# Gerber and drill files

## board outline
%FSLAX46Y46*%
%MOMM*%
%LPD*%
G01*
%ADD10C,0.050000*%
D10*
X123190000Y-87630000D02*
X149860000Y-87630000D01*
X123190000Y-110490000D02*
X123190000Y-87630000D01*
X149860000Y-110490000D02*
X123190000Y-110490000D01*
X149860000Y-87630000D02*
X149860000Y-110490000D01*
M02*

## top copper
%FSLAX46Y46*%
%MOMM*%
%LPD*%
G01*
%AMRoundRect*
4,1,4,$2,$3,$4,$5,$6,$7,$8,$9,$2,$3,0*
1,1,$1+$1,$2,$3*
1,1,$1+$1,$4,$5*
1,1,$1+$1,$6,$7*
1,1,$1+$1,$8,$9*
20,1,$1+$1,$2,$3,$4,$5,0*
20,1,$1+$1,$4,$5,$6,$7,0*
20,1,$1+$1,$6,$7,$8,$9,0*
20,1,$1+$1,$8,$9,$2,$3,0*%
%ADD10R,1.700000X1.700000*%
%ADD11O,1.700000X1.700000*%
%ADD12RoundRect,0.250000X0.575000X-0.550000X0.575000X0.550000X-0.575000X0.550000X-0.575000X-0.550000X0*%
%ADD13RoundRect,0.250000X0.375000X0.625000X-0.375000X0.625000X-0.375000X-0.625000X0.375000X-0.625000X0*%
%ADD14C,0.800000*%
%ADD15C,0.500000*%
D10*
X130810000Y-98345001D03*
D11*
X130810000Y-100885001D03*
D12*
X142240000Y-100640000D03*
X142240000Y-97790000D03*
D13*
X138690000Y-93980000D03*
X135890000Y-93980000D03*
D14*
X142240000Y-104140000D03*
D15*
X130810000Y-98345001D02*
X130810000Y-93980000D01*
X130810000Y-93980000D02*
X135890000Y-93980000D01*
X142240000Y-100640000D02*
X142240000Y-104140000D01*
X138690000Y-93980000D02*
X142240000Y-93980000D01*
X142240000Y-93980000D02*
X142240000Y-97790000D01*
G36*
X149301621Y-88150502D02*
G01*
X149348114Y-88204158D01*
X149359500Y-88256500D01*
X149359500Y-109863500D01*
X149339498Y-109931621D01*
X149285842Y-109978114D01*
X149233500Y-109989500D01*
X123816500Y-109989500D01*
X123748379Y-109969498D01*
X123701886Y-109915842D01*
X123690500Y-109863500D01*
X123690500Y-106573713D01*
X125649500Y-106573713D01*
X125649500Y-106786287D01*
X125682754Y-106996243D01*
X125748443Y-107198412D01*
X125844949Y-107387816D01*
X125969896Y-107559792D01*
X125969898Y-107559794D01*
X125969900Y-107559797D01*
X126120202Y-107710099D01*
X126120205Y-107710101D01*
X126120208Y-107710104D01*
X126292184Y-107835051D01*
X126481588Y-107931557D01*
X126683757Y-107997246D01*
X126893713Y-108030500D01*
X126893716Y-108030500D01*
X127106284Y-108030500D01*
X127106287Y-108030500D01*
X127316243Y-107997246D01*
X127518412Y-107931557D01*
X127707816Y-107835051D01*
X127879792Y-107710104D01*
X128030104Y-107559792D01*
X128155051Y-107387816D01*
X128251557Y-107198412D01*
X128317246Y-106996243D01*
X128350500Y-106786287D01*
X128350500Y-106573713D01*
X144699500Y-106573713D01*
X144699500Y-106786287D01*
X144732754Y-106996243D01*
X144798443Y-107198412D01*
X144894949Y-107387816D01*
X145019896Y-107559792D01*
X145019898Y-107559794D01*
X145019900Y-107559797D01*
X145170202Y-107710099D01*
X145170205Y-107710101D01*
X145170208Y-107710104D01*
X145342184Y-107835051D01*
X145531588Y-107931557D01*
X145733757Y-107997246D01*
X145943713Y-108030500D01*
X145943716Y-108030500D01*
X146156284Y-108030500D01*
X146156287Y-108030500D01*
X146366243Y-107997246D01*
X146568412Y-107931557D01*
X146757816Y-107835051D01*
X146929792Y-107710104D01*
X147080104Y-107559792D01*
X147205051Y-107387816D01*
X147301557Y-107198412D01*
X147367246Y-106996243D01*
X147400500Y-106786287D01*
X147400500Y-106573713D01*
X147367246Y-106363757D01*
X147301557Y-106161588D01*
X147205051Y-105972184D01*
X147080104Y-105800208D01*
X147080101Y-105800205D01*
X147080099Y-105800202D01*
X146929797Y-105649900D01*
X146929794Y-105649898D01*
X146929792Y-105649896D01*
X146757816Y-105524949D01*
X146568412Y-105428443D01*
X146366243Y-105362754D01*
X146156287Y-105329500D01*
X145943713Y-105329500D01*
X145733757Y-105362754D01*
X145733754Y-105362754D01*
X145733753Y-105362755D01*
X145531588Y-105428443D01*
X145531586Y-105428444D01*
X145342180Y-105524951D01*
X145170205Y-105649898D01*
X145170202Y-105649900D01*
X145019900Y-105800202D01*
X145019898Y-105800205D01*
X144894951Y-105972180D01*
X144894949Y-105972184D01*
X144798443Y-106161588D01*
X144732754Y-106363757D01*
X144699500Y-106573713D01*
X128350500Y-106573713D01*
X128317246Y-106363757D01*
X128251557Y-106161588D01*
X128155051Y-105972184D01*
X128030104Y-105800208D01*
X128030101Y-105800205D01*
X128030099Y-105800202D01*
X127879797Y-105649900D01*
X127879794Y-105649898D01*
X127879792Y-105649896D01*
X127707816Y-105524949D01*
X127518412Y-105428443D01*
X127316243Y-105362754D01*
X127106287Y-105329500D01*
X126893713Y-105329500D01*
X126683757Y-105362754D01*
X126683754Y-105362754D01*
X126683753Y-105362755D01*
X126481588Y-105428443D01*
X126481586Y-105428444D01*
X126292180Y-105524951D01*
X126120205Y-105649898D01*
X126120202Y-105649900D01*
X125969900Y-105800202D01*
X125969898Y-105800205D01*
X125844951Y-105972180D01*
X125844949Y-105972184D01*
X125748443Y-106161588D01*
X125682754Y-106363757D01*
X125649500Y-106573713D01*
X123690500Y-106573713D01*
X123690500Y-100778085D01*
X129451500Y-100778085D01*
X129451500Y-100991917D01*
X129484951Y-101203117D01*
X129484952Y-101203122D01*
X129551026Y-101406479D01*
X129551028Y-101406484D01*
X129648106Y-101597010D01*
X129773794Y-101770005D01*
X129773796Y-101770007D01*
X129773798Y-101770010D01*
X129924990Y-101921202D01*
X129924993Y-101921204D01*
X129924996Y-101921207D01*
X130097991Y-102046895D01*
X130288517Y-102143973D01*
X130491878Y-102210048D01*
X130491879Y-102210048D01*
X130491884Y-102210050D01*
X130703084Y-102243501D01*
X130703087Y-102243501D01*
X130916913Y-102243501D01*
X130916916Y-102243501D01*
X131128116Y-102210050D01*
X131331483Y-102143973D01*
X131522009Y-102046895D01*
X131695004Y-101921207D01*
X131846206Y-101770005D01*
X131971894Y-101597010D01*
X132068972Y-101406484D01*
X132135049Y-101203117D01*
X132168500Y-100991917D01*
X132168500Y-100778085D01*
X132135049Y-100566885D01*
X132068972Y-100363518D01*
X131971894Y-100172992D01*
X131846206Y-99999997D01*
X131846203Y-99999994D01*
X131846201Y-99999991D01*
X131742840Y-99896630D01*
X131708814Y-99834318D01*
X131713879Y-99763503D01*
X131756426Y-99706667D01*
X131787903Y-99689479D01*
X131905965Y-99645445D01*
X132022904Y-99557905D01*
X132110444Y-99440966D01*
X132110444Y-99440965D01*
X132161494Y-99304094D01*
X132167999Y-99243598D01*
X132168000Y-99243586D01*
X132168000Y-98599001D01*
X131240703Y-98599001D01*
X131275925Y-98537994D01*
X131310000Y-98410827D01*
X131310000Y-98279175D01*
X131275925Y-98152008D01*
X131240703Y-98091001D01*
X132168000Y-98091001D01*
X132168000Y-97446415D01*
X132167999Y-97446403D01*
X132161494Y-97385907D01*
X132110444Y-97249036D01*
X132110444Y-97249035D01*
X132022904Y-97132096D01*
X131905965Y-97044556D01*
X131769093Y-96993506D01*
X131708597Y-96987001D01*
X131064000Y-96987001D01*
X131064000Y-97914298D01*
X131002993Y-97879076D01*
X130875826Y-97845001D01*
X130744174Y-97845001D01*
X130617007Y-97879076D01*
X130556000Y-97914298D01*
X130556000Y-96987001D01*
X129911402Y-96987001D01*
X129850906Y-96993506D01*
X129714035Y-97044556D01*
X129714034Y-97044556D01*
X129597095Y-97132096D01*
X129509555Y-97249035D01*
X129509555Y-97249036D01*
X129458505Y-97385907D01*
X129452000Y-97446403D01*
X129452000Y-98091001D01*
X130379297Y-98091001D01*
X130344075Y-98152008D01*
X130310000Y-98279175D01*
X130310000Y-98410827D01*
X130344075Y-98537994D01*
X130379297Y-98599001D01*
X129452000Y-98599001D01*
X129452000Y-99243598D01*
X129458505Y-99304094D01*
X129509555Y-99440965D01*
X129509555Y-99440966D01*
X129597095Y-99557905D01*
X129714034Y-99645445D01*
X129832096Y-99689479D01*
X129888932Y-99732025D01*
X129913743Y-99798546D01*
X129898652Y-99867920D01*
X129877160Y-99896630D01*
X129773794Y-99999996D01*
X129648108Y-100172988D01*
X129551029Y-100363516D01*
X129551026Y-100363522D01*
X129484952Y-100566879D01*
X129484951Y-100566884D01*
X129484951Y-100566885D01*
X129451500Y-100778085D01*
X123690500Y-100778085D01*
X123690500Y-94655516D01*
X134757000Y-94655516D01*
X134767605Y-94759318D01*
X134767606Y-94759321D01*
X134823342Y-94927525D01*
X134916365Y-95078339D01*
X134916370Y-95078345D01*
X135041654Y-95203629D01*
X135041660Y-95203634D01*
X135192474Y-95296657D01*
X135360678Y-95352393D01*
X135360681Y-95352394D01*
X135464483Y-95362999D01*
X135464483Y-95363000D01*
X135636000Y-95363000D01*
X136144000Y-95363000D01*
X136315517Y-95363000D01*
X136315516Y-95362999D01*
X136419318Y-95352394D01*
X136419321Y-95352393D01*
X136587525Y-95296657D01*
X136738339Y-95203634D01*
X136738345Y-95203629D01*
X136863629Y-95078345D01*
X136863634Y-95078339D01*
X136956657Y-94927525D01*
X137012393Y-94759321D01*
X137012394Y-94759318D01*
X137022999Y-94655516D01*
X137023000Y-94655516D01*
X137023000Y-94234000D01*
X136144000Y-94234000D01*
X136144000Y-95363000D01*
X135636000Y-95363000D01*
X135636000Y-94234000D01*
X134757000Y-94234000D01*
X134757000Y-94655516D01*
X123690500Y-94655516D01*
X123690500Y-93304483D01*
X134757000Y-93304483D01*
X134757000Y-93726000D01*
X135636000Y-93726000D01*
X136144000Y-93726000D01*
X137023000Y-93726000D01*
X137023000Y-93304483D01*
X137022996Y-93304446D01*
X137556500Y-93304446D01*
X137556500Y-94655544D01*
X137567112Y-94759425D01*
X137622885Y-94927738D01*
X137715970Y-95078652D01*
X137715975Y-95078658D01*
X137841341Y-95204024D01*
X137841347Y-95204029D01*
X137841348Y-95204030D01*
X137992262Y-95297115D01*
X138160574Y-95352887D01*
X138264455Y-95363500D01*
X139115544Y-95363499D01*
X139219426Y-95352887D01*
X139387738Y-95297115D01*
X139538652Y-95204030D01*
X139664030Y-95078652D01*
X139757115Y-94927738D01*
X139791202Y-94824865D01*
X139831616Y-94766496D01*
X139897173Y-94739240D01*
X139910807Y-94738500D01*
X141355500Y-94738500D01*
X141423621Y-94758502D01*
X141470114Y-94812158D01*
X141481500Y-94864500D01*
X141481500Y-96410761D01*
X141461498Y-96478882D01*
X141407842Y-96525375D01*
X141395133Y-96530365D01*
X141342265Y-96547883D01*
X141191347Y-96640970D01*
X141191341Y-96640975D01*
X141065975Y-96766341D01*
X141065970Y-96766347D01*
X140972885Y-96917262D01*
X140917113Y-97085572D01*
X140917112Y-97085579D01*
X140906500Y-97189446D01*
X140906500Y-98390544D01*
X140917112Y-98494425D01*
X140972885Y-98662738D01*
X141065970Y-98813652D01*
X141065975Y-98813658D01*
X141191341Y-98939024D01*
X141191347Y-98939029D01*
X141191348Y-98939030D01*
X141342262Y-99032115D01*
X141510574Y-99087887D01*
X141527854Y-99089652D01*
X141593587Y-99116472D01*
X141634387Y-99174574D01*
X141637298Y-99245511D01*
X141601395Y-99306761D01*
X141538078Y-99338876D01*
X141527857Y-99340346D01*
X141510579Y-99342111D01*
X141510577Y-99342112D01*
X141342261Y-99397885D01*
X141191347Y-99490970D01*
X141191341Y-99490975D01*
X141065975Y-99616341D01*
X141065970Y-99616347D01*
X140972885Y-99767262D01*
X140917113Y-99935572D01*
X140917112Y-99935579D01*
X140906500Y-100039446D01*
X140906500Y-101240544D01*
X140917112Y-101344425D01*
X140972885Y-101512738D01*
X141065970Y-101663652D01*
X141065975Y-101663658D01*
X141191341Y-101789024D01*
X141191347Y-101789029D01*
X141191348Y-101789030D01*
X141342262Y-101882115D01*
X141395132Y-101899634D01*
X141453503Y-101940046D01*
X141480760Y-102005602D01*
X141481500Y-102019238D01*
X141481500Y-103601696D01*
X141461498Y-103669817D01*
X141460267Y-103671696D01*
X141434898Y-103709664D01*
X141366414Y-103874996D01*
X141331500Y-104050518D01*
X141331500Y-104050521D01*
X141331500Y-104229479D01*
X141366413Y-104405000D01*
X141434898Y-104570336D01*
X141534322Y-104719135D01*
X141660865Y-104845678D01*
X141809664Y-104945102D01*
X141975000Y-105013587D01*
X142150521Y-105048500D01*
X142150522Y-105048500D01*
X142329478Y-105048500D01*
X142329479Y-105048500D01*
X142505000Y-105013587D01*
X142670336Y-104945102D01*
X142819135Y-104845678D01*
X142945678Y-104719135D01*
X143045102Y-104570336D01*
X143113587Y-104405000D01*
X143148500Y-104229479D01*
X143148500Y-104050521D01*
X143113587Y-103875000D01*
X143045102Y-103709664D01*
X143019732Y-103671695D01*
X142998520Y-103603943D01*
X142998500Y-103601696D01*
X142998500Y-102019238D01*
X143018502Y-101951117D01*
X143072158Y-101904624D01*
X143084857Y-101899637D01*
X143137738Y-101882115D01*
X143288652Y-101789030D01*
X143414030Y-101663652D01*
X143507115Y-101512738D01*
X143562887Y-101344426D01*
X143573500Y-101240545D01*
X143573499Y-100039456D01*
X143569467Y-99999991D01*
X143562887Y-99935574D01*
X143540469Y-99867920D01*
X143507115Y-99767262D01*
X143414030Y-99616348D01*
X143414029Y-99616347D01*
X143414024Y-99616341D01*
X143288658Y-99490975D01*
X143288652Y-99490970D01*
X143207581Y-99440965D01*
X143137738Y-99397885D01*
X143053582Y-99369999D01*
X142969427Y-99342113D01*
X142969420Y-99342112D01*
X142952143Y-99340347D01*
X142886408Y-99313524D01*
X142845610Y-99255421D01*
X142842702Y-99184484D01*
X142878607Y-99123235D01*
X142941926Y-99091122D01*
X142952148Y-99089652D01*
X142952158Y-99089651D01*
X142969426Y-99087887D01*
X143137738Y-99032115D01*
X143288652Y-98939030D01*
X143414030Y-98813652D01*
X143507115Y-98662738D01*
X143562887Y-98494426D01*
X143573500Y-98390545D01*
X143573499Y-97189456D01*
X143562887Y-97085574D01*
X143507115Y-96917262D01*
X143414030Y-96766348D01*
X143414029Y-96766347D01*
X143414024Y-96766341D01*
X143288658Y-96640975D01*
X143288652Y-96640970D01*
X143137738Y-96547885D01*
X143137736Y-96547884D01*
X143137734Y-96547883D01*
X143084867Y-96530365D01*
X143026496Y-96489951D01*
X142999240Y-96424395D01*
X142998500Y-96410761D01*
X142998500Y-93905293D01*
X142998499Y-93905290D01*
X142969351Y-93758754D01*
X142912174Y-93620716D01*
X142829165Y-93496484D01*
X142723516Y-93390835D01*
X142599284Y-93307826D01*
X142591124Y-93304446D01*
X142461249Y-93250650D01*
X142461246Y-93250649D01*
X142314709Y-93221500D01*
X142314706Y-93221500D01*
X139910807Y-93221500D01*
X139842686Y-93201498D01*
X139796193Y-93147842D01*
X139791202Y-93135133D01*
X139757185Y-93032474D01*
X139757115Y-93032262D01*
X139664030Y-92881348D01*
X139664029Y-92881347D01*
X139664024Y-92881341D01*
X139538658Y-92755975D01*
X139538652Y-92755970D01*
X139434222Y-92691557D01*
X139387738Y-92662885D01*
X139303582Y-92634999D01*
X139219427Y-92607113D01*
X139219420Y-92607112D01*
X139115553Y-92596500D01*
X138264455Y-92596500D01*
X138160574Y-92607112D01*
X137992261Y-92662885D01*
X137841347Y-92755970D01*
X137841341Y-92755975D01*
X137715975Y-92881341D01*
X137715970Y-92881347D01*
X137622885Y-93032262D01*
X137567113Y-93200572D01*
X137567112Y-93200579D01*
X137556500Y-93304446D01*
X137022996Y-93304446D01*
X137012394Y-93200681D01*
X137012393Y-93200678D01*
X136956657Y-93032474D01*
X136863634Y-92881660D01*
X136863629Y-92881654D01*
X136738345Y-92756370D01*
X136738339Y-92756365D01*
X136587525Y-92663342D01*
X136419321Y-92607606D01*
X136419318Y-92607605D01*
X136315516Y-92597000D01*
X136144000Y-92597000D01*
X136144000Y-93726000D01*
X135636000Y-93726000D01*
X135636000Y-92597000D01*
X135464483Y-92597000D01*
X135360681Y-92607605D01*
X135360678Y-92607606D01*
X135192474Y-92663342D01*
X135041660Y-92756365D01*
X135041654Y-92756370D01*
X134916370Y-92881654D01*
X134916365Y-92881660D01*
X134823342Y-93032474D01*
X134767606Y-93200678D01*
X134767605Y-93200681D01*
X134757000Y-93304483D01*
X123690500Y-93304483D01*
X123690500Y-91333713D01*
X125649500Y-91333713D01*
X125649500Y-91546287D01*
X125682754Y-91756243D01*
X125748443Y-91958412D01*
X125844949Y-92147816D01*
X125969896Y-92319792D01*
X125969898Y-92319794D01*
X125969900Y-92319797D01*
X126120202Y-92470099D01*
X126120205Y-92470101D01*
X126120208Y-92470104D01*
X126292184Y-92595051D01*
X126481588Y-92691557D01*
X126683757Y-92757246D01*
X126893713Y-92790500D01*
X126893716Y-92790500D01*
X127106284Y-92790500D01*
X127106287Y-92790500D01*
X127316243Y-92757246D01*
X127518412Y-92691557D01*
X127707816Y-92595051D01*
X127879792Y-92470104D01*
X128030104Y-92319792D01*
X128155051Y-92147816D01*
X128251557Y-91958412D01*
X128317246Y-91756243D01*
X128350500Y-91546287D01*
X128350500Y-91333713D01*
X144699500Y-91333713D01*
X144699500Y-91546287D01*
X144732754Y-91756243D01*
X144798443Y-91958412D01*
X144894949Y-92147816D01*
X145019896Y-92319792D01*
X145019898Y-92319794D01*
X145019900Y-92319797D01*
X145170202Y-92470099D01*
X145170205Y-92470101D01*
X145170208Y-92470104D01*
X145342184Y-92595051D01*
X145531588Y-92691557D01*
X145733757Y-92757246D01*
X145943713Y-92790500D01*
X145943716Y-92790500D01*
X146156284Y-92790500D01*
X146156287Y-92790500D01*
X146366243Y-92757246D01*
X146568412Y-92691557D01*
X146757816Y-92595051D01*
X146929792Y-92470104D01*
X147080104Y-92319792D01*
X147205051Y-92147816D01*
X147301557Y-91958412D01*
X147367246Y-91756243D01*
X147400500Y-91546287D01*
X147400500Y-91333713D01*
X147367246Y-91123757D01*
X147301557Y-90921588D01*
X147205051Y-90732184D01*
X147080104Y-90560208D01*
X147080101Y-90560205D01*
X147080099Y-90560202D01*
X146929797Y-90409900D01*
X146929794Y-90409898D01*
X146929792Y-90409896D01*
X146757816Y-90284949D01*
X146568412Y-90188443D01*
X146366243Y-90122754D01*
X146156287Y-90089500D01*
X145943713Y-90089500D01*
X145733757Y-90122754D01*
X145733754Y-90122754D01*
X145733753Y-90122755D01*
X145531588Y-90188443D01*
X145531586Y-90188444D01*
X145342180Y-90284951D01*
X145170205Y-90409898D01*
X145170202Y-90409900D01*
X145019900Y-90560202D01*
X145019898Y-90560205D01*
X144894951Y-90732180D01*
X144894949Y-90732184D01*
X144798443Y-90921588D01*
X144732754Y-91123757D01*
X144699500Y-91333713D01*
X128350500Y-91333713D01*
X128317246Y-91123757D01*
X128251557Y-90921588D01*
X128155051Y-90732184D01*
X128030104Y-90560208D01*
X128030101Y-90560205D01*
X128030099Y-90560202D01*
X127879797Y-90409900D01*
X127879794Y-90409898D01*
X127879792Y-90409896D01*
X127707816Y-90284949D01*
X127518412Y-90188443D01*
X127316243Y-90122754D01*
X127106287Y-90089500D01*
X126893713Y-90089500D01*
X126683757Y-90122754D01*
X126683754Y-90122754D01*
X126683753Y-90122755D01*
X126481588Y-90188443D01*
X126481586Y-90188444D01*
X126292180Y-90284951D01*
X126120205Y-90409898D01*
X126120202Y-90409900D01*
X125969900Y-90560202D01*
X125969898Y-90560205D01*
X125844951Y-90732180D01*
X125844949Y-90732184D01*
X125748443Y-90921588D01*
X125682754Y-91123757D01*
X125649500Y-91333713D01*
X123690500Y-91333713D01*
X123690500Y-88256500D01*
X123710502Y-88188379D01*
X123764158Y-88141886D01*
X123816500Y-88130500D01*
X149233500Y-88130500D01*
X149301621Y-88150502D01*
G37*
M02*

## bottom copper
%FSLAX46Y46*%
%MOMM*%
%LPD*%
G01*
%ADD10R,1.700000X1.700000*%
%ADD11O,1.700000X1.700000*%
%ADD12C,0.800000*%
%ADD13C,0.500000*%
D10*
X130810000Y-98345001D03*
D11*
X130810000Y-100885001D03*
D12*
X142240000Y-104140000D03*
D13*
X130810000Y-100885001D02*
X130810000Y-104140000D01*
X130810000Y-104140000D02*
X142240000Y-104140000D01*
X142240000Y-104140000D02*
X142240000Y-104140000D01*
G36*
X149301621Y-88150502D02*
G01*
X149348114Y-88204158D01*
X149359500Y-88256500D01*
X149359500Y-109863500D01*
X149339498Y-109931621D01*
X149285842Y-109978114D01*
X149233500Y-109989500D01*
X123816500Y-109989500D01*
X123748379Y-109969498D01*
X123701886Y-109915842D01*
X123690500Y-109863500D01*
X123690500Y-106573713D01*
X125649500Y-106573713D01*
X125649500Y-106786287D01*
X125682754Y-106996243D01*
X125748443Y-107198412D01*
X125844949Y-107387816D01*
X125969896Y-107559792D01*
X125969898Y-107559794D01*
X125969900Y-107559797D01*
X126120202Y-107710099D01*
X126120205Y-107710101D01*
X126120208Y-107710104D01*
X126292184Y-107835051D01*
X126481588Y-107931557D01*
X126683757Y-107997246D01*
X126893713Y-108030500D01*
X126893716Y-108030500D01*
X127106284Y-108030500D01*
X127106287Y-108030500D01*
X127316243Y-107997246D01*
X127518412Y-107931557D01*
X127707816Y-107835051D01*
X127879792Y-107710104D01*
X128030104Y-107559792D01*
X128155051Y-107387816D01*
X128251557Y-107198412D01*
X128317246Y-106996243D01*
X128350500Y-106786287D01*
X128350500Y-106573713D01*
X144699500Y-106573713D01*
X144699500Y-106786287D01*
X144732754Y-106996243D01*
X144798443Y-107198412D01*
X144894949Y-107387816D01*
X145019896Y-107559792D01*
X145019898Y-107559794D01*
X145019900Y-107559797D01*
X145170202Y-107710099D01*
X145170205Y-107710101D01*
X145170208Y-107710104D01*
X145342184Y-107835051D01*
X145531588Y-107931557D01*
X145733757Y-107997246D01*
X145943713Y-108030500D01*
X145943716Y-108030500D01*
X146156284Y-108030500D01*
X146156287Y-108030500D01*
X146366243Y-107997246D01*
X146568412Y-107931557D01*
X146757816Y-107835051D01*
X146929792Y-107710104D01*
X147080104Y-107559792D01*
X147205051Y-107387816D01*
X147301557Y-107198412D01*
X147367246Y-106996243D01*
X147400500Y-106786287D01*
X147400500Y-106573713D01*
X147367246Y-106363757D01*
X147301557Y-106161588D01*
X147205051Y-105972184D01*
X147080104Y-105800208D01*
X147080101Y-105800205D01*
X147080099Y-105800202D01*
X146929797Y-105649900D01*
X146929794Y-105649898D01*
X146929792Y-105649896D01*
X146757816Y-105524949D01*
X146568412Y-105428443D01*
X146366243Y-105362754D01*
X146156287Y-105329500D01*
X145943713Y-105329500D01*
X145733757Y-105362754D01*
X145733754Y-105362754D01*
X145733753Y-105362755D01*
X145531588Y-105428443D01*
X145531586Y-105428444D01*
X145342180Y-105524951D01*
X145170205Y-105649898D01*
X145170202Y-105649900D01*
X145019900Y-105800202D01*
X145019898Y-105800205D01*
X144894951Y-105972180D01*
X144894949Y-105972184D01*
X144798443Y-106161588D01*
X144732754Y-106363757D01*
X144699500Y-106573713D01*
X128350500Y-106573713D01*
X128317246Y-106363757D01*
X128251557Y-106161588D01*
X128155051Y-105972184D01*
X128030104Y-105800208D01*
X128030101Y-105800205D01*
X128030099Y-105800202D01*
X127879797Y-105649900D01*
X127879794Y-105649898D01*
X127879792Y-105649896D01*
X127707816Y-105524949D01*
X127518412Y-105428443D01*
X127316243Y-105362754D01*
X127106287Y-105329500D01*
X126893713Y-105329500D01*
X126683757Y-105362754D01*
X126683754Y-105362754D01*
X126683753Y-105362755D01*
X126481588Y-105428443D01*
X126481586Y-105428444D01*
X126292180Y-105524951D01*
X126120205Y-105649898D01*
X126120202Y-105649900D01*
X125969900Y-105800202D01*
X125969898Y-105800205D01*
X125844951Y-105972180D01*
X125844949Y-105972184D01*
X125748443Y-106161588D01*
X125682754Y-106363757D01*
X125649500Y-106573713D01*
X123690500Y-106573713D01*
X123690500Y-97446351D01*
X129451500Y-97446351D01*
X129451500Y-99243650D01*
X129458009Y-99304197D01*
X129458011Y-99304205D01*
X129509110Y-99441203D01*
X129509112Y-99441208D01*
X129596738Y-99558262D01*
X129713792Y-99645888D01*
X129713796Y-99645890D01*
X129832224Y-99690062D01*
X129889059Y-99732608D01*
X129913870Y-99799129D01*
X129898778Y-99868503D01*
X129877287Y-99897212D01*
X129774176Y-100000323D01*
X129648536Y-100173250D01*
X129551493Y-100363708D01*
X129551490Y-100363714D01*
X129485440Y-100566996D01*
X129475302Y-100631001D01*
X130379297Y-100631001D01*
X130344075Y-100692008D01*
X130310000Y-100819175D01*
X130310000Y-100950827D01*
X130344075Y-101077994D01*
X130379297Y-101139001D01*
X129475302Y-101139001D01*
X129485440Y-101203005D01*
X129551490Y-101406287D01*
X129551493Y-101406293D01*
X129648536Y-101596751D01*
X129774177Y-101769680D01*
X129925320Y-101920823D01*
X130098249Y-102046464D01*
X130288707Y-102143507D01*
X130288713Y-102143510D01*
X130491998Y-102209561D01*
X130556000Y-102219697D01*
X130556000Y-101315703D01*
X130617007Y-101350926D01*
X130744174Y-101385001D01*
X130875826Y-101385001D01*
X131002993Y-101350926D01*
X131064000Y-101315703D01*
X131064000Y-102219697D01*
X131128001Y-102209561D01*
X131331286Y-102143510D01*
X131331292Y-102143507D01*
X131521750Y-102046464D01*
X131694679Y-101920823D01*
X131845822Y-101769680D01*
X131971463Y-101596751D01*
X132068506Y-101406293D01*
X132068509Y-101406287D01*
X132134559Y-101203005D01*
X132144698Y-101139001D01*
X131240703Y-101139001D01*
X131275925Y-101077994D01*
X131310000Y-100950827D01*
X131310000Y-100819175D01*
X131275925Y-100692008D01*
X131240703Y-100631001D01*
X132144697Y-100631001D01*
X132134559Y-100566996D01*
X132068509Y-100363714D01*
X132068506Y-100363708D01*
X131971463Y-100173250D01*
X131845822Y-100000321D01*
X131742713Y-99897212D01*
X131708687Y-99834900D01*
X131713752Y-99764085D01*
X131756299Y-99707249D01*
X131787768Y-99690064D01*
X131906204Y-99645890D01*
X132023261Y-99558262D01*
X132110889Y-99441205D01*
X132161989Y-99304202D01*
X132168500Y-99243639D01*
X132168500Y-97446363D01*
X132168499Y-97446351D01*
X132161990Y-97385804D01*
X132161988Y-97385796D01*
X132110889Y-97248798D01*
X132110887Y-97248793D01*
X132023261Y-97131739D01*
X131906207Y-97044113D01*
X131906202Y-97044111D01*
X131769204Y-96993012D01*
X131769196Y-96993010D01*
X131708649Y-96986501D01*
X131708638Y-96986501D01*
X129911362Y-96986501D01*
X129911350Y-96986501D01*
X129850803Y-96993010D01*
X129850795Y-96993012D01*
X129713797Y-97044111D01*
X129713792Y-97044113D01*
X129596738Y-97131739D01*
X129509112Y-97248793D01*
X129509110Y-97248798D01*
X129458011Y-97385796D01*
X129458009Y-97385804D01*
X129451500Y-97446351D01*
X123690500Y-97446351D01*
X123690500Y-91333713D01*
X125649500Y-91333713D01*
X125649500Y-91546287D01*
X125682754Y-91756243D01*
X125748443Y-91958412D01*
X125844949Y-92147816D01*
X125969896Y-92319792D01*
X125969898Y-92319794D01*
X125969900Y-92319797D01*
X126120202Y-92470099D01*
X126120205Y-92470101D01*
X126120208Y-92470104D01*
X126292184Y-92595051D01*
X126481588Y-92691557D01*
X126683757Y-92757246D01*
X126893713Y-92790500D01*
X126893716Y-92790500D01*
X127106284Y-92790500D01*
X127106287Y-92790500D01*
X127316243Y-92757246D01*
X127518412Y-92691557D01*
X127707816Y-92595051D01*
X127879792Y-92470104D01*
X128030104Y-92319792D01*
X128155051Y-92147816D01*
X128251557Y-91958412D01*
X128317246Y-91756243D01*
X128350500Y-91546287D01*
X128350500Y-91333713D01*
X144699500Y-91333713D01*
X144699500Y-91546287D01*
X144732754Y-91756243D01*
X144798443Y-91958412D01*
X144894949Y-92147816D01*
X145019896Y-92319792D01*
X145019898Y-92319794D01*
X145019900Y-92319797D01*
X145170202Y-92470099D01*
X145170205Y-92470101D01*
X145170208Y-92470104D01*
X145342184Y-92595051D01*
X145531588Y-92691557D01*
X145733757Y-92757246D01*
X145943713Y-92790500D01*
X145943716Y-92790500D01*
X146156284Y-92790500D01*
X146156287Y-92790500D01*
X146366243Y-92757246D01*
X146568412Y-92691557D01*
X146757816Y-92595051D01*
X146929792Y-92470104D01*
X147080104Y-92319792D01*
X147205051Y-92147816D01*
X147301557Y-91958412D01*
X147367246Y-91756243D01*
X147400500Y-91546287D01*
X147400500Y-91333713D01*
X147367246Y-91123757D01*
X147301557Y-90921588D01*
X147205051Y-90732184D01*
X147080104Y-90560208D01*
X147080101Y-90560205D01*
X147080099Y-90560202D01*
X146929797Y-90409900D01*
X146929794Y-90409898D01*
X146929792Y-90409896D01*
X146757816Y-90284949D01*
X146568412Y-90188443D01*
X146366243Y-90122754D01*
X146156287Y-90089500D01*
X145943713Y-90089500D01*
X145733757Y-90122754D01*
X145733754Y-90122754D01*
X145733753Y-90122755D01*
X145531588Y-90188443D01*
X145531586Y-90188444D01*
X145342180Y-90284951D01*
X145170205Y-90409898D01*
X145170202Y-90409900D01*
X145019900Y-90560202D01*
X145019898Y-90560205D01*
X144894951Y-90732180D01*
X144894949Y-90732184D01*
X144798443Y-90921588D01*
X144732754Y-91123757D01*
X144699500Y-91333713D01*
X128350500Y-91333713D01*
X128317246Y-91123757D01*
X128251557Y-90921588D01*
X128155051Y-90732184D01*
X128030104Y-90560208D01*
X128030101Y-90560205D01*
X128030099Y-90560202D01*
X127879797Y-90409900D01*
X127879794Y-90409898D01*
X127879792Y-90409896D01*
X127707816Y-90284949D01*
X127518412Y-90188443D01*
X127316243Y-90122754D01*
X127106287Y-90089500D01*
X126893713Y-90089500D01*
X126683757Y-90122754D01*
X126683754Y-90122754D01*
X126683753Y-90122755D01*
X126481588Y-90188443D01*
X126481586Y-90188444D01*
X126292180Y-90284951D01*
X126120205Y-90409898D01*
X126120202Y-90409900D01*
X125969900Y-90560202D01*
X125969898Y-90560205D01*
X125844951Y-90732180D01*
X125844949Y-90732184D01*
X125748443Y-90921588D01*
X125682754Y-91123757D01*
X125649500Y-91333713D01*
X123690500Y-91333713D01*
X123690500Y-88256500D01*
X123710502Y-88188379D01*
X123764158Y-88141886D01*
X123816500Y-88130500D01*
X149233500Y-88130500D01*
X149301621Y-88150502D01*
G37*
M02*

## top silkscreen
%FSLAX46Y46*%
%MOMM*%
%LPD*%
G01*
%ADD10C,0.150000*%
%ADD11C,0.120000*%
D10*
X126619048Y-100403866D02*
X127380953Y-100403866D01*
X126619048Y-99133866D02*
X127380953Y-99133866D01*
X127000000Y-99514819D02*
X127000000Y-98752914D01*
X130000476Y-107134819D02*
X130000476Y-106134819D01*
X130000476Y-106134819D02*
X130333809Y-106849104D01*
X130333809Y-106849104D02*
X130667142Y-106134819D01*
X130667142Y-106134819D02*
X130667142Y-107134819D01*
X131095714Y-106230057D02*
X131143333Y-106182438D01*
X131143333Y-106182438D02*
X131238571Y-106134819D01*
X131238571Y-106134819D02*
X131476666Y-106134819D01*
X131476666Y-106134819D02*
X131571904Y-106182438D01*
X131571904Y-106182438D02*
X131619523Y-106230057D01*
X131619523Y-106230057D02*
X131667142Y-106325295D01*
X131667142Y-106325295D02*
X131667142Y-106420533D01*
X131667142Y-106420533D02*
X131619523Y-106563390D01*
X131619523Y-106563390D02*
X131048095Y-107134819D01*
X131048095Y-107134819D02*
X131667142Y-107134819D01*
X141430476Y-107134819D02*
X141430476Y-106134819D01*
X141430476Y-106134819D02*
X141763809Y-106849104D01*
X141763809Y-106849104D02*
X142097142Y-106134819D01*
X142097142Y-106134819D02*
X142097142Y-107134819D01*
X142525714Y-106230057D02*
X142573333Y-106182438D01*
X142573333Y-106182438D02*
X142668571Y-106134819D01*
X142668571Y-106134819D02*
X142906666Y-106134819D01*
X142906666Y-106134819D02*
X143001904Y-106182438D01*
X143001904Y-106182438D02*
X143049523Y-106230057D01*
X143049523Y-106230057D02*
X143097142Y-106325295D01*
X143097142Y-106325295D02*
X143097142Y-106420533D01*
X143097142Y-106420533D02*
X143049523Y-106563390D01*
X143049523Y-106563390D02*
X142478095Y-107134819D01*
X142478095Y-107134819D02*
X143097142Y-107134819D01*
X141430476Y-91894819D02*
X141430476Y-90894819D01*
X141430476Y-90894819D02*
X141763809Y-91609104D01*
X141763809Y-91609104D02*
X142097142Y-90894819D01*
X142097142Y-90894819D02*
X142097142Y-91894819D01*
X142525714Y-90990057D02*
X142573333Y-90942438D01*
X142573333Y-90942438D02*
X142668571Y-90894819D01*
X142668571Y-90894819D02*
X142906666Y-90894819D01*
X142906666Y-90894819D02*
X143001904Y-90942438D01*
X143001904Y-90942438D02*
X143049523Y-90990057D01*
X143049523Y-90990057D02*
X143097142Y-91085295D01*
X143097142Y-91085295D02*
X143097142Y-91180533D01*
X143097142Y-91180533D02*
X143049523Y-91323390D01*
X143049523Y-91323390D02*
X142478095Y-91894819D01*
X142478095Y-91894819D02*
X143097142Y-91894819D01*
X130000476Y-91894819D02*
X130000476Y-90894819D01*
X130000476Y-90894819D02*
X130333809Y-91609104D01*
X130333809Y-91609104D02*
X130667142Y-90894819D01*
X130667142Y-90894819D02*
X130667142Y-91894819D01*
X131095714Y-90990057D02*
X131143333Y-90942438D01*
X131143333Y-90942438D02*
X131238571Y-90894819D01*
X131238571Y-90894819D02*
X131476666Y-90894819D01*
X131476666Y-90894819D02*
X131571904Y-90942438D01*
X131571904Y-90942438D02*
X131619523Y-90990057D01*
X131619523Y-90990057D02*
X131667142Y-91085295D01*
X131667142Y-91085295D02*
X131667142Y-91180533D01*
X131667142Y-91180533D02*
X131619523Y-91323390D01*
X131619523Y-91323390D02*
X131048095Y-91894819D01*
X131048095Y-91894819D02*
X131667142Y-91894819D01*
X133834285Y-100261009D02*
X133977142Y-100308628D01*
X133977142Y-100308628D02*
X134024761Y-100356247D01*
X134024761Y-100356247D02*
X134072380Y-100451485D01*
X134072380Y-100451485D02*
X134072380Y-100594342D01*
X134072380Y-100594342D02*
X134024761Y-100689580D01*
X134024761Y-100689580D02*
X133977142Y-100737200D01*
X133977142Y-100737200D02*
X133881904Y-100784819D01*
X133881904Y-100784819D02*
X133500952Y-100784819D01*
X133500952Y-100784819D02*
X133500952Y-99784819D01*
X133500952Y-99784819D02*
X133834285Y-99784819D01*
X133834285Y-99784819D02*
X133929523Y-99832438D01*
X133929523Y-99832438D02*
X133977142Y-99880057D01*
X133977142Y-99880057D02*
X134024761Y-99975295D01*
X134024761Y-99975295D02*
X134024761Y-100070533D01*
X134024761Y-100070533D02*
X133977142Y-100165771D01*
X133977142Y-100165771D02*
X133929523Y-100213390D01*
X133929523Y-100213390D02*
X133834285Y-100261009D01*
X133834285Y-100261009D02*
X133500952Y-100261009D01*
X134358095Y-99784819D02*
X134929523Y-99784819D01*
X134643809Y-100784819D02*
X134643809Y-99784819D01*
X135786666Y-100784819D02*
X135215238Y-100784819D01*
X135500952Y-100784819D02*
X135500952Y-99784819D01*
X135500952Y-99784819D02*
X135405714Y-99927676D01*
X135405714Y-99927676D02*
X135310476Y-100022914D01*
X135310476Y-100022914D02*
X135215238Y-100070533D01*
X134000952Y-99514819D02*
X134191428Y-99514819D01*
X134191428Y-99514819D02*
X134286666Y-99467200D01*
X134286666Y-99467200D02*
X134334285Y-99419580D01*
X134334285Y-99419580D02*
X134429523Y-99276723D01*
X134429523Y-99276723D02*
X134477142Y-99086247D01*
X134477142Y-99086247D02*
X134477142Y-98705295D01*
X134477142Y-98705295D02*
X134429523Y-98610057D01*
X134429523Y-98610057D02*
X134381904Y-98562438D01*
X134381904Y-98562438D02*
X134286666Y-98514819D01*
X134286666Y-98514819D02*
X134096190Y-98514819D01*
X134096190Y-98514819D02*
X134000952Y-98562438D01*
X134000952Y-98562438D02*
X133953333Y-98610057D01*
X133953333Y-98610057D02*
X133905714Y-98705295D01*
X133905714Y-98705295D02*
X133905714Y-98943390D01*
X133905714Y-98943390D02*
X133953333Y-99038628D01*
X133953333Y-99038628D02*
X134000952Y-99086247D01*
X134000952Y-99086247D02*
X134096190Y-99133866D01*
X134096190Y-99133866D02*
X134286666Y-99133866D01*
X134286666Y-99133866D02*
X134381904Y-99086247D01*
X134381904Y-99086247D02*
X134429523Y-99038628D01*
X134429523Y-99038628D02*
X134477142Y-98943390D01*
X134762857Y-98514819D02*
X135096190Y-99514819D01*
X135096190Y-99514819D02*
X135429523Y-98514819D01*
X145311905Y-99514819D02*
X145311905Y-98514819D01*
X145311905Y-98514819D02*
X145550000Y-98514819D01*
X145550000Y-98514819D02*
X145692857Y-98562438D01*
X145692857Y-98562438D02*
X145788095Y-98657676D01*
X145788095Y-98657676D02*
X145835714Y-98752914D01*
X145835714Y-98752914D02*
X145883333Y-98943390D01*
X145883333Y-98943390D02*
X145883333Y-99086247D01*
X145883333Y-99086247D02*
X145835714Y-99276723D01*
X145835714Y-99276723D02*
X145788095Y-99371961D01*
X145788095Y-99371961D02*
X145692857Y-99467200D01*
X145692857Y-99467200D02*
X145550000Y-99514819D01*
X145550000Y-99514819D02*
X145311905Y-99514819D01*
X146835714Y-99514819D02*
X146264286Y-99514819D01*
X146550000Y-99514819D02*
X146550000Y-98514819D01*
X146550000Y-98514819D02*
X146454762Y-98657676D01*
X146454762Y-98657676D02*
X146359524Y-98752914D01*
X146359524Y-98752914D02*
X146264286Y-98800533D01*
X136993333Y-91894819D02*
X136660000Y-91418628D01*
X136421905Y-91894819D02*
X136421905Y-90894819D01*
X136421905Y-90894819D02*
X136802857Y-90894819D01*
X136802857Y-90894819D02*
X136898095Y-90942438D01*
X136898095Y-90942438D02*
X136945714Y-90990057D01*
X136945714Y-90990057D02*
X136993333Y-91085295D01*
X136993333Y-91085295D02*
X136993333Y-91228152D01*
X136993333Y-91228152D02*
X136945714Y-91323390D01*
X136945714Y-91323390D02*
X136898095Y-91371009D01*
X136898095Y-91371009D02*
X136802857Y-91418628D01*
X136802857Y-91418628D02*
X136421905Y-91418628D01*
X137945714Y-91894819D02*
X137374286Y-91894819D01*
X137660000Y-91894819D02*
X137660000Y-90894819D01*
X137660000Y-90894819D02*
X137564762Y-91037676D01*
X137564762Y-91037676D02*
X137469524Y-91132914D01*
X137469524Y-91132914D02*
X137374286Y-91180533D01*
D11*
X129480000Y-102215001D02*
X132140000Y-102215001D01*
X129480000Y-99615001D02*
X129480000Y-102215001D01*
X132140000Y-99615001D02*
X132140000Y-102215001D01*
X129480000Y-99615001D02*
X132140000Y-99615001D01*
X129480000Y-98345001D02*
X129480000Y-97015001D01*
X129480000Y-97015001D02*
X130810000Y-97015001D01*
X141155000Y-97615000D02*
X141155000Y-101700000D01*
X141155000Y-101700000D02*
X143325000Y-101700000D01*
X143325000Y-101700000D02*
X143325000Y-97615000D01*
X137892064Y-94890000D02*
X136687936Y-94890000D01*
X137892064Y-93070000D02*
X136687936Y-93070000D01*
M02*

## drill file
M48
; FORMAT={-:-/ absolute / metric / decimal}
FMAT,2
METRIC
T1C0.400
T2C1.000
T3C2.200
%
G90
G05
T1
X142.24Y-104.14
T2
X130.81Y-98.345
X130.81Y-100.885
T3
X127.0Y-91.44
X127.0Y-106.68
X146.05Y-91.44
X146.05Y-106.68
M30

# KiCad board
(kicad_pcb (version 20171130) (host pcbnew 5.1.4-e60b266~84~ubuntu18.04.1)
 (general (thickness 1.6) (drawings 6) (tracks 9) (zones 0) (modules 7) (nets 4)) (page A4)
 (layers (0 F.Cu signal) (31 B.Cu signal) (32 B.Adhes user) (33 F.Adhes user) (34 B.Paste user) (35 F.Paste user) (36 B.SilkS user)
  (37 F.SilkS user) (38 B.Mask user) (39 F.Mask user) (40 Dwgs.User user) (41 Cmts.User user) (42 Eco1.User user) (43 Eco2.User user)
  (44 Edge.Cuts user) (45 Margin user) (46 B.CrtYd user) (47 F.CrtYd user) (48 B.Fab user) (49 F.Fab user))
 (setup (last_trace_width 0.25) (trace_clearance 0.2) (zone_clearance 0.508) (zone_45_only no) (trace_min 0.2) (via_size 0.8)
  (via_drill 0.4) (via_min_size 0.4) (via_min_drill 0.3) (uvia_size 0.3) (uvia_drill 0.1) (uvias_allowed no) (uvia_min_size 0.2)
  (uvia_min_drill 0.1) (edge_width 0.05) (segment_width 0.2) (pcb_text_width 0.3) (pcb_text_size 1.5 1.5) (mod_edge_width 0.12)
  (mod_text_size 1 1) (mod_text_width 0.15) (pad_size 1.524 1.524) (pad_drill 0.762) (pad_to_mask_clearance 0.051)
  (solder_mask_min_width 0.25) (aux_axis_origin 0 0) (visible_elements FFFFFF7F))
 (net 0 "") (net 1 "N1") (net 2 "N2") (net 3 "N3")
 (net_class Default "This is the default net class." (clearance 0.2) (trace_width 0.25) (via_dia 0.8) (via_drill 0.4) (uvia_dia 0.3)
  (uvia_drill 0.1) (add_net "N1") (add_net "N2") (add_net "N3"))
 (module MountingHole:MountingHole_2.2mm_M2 (layer F.Cu) (at 127 106.68)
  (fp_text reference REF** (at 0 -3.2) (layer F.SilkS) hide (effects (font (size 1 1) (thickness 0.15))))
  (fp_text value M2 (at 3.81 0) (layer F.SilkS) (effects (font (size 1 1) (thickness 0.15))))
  (pad 1 np_thru_hole circle (at 0 0) (size 2.2 2.2) (drill 2.2) (layers *.Cu *.Mask)))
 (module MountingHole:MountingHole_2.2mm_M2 (layer F.Cu) (at 146.05 106.68)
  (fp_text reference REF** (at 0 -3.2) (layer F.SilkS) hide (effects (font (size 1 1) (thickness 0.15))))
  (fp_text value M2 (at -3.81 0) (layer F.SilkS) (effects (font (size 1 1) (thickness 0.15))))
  (pad 1 np_thru_hole circle (at 0 0) (size 2.2 2.2) (drill 2.2) (layers *.Cu *.Mask)))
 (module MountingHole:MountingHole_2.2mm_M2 (layer F.Cu) (at 146.05 91.44)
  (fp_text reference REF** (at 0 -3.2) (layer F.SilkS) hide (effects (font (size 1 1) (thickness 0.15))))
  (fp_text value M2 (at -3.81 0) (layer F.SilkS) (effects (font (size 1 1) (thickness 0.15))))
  (pad 1 np_thru_hole circle (at 0 0) (size 2.2 2.2) (drill 2.2) (layers *.Cu *.Mask)))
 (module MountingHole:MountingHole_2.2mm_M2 (layer B.Cu) (at 127 91.44)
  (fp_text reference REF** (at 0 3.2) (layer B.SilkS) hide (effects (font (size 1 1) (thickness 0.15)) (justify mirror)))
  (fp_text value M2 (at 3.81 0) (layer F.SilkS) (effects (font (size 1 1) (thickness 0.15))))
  (pad 1 np_thru_hole circle (at 0 0) (size 2.2 2.2) (drill 2.2) (layers *.Cu *.Mask)))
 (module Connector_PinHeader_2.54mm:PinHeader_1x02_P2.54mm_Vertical (layer F.Cu) (at 130.81 98.345001)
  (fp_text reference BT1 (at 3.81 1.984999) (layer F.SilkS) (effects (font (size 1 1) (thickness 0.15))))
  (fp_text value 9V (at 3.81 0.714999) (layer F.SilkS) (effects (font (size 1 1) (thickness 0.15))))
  (fp_line (start -1.33 3.87) (end 1.33 3.87) (layer F.SilkS) (width 0.12))
  (fp_line (start -1.33 1.27) (end -1.33 3.87) (layer F.SilkS) (width 0.12))
  (fp_line (start 1.33 1.27) (end 1.33 3.87) (layer F.SilkS) (width 0.12))
  (fp_line (start -1.33 1.27) (end 1.33 1.27) (layer F.SilkS) (width 0.12))
  (fp_line (start -1.33 0) (end -1.33 -1.33) (layer F.SilkS) (width 0.12))
  (fp_line (start -1.33 -1.33) (end 0 -1.33) (layer F.SilkS) (width 0.12))
  (pad 1 thru_hole rect (at 0 0) (size 1.7 1.7) (drill 1) (layers *.Cu *.Mask) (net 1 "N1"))
  (pad 2 thru_hole oval (at 0 2.54) (size 1.7 1.7) (drill 1) (layers *.Cu *.Mask) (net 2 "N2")))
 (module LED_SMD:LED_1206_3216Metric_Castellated (layer F.Cu) (at 142.24 99.215 90)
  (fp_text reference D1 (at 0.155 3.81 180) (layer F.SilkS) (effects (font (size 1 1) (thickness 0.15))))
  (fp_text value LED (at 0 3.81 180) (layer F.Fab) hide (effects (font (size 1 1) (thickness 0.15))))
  (fp_line (start 1.6 -1.085) (end -2.485 -1.085) (layer F.SilkS) (width 0.12))
  (fp_line (start -2.485 -1.085) (end -2.485 1.085) (layer F.SilkS) (width 0.12))
  (fp_line (start -2.485 1.085) (end 1.6 1.085) (layer F.SilkS) (width 0.12))
  (pad 1 smd roundrect (at -1.425 0 90) (size 1.6 1.65) (layers F.Cu F.Paste F.Mask) (roundrect_rratio 0.15625) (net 2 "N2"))
  (pad 2 smd roundrect (at 1.425 0 90) (size 1.6 1.65) (layers F.Cu F.Paste F.Mask) (roundrect_rratio 0.15625) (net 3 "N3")))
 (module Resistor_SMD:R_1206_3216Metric (layer F.Cu) (at 137.29 93.98 180)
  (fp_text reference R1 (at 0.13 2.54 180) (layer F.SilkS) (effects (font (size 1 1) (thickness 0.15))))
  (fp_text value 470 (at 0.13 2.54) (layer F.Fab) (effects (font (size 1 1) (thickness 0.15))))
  (fp_line (start -0.602064 -0.91) (end 0.602064 -0.91) (layer F.SilkS) (width 0.12))
  (fp_line (start -0.602064 0.91) (end 0.602064 0.91) (layer F.SilkS) (width 0.12))
  (pad 1 smd roundrect (at -1.4 0 180) (size 1.25 1.75) (layers F.Cu F.Paste F.Mask) (roundrect_rratio 0.2) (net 3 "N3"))
  (pad 2 smd roundrect (at 1.4 0 180) (size 1.25 1.75) (layers F.Cu F.Paste F.Mask) (roundrect_rratio 0.2) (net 1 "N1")))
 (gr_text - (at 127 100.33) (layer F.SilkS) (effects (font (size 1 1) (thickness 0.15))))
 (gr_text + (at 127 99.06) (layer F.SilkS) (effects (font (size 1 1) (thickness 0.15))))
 (gr_line (start 123.19 87.63) (end 149.86 87.63) (layer Edge.Cuts) (width 0.05))
 (gr_line (start 123.19 110.49) (end 123.19 87.63) (layer Edge.Cuts) (width 0.05))
 (gr_line (start 149.86 110.49) (end 123.19 110.49) (layer Edge.Cuts) (width 0.05))
 (gr_line (start 149.86 87.63) (end 149.86 110.49) (layer Edge.Cuts) (width 0.05))
 (segment (start 130.81 98.345001) (end 130.81 93.98) (width 0.5) (layer F.Cu) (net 1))
 (segment (start 130.81 93.98) (end 135.89 93.98) (width 0.5) (layer F.Cu) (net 1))
 (segment (start 130.81 100.885001) (end 130.81 104.14) (width 0.5) (layer B.Cu) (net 2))
 (segment (start 130.81 104.14) (end 142.24 104.14) (width 0.5) (layer B.Cu) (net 2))
 (segment (start 142.24 104.14) (end 142.24 104.14) (width 0.5) (layer B.Cu) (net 2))
 (via (at 142.24 104.14) (size 0.8) (drill 0.4) (layers F.Cu B.Cu) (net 2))
 (segment (start 142.24 100.64) (end 142.24 104.14) (width 0.5) (layer F.Cu) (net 2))
 (segment (start 138.69 93.98) (end 142.24 93.98) (width 0.5) (layer F.Cu) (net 3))
 (segment (start 142.24 93.98) (end 142.24 97.79) (width 0.5) (layer F.Cu) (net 3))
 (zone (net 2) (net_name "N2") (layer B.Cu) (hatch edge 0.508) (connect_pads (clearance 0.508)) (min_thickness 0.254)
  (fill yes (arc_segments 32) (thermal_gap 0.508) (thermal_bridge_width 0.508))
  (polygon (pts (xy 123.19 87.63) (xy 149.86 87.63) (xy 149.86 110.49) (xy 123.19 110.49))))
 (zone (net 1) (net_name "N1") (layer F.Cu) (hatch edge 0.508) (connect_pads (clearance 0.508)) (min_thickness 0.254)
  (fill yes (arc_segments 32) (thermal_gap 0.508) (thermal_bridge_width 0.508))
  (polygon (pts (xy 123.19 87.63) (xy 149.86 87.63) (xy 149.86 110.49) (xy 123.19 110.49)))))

